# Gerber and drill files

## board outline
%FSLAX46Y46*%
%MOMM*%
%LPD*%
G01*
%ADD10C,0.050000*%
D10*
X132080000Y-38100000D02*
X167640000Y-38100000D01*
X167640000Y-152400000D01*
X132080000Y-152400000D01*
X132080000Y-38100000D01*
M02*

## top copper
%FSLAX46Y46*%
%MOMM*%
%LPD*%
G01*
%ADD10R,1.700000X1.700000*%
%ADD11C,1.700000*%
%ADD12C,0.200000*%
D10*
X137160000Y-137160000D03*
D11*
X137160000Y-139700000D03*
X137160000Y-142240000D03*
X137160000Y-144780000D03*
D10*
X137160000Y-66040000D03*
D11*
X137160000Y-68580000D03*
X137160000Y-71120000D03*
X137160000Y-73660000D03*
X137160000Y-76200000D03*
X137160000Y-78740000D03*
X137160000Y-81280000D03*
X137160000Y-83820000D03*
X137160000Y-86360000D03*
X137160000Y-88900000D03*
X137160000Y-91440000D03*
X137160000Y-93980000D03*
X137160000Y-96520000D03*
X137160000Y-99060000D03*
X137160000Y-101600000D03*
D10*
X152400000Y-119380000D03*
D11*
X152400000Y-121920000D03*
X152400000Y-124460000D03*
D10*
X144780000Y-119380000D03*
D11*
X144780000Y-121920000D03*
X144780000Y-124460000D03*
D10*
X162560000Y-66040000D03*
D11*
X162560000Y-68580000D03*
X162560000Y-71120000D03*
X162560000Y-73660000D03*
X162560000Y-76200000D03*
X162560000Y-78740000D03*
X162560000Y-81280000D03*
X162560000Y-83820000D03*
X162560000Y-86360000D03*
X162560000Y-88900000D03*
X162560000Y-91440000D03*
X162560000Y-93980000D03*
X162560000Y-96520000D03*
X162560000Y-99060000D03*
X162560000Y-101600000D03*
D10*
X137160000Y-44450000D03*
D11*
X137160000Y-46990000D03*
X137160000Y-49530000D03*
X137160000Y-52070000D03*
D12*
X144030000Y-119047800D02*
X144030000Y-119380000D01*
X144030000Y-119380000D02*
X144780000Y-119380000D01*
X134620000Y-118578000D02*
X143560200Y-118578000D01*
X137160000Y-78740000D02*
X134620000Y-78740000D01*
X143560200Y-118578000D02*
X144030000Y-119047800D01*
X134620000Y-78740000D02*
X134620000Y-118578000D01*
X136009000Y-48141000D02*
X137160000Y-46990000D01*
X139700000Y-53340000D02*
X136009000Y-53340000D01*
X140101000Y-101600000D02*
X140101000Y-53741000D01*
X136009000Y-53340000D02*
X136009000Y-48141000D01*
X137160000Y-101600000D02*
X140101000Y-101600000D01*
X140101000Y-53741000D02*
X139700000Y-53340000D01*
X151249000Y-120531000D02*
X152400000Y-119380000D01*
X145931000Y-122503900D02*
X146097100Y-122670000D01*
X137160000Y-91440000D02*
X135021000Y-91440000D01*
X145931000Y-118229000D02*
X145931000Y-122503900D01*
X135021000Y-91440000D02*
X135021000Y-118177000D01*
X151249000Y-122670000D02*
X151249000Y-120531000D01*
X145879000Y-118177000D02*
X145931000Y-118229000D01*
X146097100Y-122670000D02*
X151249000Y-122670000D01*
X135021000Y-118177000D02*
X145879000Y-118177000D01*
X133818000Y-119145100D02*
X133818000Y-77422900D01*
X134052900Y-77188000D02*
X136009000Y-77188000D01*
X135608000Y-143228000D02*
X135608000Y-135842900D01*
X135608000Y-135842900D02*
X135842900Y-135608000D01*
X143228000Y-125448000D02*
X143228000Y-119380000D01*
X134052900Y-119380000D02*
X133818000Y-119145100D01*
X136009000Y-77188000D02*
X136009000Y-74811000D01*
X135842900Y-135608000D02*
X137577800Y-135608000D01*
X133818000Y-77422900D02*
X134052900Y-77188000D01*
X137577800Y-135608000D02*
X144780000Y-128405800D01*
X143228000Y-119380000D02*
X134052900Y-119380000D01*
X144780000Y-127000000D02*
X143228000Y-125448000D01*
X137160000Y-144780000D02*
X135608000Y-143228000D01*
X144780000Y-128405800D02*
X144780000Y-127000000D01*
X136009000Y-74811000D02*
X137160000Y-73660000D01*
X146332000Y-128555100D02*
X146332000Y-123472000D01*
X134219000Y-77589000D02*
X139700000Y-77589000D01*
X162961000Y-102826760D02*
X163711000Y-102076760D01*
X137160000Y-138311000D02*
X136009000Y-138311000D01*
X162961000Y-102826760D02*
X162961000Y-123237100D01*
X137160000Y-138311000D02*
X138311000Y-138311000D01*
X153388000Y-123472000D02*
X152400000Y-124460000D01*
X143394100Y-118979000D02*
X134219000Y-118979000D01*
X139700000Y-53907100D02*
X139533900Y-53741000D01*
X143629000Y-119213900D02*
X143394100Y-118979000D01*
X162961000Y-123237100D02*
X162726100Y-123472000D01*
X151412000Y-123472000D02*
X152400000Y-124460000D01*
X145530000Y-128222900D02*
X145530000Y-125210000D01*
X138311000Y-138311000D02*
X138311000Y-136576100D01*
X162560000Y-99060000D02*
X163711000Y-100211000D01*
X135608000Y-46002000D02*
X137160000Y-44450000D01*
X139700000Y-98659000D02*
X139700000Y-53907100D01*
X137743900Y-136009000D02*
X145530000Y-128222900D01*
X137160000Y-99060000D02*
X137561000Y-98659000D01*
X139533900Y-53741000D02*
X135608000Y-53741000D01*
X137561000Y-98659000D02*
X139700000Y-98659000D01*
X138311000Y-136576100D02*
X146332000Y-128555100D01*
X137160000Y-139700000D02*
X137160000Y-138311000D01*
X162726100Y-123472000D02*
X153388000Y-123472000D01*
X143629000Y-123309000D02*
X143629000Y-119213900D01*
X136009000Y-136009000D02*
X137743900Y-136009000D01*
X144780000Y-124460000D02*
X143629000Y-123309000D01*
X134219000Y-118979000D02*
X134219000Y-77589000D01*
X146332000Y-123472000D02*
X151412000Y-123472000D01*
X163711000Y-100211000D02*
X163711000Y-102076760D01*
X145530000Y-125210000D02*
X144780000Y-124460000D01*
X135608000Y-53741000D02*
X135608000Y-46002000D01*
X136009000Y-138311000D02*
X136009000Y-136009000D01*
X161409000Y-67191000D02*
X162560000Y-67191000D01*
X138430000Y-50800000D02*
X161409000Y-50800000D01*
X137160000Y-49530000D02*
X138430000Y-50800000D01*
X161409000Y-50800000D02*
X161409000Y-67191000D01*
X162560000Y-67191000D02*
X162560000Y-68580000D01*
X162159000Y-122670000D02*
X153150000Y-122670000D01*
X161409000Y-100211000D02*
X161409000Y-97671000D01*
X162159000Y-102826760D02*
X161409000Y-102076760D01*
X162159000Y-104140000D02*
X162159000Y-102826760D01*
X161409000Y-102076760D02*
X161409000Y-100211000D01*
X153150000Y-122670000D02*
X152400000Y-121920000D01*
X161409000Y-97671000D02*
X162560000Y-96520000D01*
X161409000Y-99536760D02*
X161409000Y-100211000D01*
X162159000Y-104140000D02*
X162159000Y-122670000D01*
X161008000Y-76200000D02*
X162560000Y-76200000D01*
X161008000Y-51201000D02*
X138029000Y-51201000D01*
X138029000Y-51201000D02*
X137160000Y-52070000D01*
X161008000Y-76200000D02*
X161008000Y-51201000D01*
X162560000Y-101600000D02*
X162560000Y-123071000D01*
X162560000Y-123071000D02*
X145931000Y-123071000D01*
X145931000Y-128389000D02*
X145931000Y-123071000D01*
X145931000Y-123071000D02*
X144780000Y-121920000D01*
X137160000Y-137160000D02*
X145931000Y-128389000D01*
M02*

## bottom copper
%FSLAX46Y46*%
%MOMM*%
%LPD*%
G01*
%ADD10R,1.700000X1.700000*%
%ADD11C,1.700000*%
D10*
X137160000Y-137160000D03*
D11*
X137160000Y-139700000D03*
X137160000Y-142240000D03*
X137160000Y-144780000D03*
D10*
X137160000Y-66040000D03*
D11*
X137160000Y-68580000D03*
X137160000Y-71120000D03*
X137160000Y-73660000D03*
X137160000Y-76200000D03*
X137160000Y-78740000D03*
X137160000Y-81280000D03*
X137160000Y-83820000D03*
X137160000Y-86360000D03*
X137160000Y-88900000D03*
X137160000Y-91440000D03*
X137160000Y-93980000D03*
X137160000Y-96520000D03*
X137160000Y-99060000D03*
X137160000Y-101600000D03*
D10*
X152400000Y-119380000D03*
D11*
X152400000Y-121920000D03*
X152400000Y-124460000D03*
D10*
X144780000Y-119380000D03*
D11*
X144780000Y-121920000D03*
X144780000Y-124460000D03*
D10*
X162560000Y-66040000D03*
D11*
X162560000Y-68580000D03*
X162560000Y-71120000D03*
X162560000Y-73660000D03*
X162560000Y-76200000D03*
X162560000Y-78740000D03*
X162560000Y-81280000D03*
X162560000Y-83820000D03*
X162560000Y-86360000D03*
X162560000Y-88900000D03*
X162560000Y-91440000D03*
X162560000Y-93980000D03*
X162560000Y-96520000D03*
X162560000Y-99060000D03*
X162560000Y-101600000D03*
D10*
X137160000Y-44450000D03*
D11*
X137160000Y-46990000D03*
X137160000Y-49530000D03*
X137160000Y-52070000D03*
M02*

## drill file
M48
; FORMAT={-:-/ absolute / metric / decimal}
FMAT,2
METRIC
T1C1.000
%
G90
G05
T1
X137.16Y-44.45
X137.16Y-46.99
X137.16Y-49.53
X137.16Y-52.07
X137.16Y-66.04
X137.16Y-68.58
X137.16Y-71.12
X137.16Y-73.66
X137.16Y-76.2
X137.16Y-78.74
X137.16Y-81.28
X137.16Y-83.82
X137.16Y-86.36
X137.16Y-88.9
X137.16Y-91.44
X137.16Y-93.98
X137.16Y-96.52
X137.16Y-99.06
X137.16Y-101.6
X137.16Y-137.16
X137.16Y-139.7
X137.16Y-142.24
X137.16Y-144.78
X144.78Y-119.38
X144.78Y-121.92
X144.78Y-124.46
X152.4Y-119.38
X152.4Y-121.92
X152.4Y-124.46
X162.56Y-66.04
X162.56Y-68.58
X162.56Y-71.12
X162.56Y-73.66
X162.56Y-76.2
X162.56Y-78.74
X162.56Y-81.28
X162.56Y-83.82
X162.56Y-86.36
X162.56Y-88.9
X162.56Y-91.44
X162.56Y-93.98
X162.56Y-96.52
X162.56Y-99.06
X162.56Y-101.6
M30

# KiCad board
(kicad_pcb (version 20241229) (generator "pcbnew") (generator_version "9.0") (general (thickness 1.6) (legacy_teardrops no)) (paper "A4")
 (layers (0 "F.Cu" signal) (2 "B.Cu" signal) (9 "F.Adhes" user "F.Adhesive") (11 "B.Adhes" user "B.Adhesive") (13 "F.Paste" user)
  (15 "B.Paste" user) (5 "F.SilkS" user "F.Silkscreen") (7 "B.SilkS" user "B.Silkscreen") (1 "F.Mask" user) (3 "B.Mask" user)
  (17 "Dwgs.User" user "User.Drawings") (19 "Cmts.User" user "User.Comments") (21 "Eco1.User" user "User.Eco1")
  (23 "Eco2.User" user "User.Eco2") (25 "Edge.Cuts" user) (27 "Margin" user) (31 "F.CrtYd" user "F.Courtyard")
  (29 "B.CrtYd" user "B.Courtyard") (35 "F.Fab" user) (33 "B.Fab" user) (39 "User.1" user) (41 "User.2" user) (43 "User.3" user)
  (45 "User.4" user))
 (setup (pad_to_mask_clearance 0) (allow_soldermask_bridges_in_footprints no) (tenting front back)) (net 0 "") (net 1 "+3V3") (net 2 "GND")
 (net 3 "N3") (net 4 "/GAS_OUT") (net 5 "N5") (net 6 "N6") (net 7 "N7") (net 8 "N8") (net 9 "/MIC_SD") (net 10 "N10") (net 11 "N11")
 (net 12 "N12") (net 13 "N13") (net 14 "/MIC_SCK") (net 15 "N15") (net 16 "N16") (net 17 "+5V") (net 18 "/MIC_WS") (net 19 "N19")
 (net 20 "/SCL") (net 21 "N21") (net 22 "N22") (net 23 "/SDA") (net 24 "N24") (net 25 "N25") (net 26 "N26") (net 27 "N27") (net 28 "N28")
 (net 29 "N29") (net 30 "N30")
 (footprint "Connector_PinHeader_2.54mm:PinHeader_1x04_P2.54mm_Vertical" (layer "F.Cu") (at 137.16 137.16)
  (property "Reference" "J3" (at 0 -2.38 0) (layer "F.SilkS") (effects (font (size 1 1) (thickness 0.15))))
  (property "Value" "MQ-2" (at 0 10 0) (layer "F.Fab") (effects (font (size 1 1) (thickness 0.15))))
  (pad "1" thru_hole rect (at 0 0) (size 1.7 1.7) (drill 1) (layers "*.Cu" "*.Mask") (remove_unused_layers no) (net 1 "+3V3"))
  (pad "2" thru_hole circle (at 0 2.54) (size 1.7 1.7) (drill 1) (layers "*.Cu" "*.Mask") (remove_unused_layers no) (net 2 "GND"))
  (pad "3" thru_hole circle (at 0 5.08) (size 1.7 1.7) (drill 1) (layers "*.Cu" "*.Mask") (remove_unused_layers no) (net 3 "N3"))
  (pad "4" thru_hole circle (at 0 7.62) (size 1.7 1.7) (drill 1) (layers "*.Cu" "*.Mask") (remove_unused_layers no) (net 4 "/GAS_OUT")))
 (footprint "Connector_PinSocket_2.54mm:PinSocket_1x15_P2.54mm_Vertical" (layer "F.Cu") (at 137.16 66.04)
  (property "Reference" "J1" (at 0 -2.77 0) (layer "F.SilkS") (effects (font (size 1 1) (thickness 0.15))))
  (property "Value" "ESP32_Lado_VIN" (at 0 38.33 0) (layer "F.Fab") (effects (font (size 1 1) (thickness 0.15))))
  (pad "1" thru_hole rect (at 0 0) (size 1.7 1.7) (drill 1) (layers "*.Cu" "*.Mask") (remove_unused_layers no) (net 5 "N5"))
  (pad "2" thru_hole circle (at 0 2.54) (size 1.7 1.7) (drill 1) (layers "*.Cu" "*.Mask") (remove_unused_layers no) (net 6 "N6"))
  (pad "3" thru_hole circle (at 0 5.08) (size 1.7 1.7) (drill 1) (layers "*.Cu" "*.Mask") (remove_unused_layers no) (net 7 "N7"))
  (pad "4" thru_hole circle (at 0 7.62) (size 1.7 1.7) (drill 1) (layers "*.Cu" "*.Mask") (remove_unused_layers no) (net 4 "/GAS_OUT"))
  (pad "5" thru_hole circle (at 0 10.16) (size 1.7 1.7) (drill 1) (layers "*.Cu" "*.Mask") (remove_unused_layers no) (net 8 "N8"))
  (pad "6" thru_hole circle (at 0 12.7) (size 1.7 1.7) (drill 1) (layers "*.Cu" "*.Mask") (remove_unused_layers no) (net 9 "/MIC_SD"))
  (pad "7" thru_hole circle (at 0 15.24) (size 1.7 1.7) (drill 1) (layers "*.Cu" "*.Mask") (remove_unused_layers no) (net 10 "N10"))
  (pad "8" thru_hole circle (at 0 17.78) (size 1.7 1.7) (drill 1) (layers "*.Cu" "*.Mask") (remove_unused_layers no) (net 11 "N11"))
  (pad "9" thru_hole circle (at 0 20.32) (size 1.7 1.7) (drill 1) (layers "*.Cu" "*.Mask") (remove_unused_layers no) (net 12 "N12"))
  (pad "10" thru_hole circle (at 0 22.86) (size 1.7 1.7) (drill 1) (layers "*.Cu" "*.Mask") (remove_unused_layers no) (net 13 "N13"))
  (pad "11" thru_hole circle (at 0 25.4) (size 1.7 1.7) (drill 1) (layers "*.Cu" "*.Mask") (remove_unused_layers no) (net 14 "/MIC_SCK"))
  (pad "12" thru_hole circle (at 0 27.94) (size 1.7 1.7) (drill 1) (layers "*.Cu" "*.Mask") (remove_unused_layers no) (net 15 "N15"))
  (pad "13" thru_hole circle (at 0 30.48) (size 1.7 1.7) (drill 1) (layers "*.Cu" "*.Mask") (remove_unused_layers no) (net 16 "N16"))
  (pad "14" thru_hole circle (at 0 33.02) (size 1.7 1.7) (drill 1) (layers "*.Cu" "*.Mask") (remove_unused_layers no) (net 2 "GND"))
  (pad "15" thru_hole circle (at 0 35.56) (size 1.7 1.7) (drill 1) (layers "*.Cu" "*.Mask") (remove_unused_layers no) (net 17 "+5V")))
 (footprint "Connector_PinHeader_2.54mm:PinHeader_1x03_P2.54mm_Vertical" (layer "F.Cu") (at 152.4 119.38)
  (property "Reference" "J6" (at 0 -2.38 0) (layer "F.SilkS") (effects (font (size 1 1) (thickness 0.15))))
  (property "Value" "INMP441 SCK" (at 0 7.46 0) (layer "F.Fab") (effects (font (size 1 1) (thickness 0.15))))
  (pad "1" thru_hole rect (at 0 0) (size 1.7 1.7) (drill 1) (layers "*.Cu" "*.Mask") (remove_unused_layers no) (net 14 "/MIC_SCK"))
  (pad "2" thru_hole circle (at 0 2.54) (size 1.7 1.7) (drill 1) (layers "*.Cu" "*.Mask") (remove_unused_layers no) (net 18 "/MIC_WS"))
  (pad "3" thru_hole circle (at 0 5.08) (size 1.7 1.7) (drill 1) (layers "*.Cu" "*.Mask") (remove_unused_layers no) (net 2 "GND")))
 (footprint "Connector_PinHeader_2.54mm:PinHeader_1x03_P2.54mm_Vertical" (layer "F.Cu") (at 144.78 119.38)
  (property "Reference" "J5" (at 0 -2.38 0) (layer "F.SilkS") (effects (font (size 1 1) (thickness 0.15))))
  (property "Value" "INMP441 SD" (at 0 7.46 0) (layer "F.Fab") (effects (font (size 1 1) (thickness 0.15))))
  (pad "1" thru_hole rect (at 0 0) (size 1.7 1.7) (drill 1) (layers "*.Cu" "*.Mask") (remove_unused_layers no) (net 9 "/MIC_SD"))
  (pad "2" thru_hole circle (at 0 2.54) (size 1.7 1.7) (drill 1) (layers "*.Cu" "*.Mask") (remove_unused_layers no) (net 1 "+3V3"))
  (pad "3" thru_hole circle (at 0 5.08) (size 1.7 1.7) (drill 1) (layers "*.Cu" "*.Mask") (remove_unused_layers no) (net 2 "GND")))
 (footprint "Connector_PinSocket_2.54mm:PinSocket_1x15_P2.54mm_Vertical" (layer "F.Cu") (at 162.56 66.04)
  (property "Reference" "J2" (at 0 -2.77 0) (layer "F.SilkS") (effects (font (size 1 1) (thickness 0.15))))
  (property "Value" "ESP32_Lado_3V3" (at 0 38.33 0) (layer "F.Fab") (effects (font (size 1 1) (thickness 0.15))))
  (pad "1" thru_hole rect (at 0 0) (size 1.7 1.7) (drill 1) (layers "*.Cu" "*.Mask") (remove_unused_layers no) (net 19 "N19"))
  (pad "2" thru_hole circle (at 0 2.54) (size 1.7 1.7) (drill 1) (layers "*.Cu" "*.Mask") (remove_unused_layers no) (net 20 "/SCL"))
  (pad "3" thru_hole circle (at 0 5.08) (size 1.7 1.7) (drill 1) (layers "*.Cu" "*.Mask") (remove_unused_layers no) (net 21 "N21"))
  (pad "4" thru_hole circle (at 0 7.62) (size 1.7 1.7) (drill 1) (layers "*.Cu" "*.Mask") (remove_unused_layers no) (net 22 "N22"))
  (pad "5" thru_hole circle (at 0 10.16) (size 1.7 1.7) (drill 1) (layers "*.Cu" "*.Mask") (remove_unused_layers no) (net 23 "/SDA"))
  (pad "6" thru_hole circle (at 0 12.7) (size 1.7 1.7) (drill 1) (layers "*.Cu" "*.Mask") (remove_unused_layers no) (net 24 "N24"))
  (pad "7" thru_hole circle (at 0 15.24) (size 1.7 1.7) (drill 1) (layers "*.Cu" "*.Mask") (remove_unused_layers no) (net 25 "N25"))
  (pad "8" thru_hole circle (at 0 17.78) (size 1.7 1.7) (drill 1) (layers "*.Cu" "*.Mask") (remove_unused_layers no) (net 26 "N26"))
  (pad "9" thru_hole circle (at 0 20.32) (size 1.7 1.7) (drill 1) (layers "*.Cu" "*.Mask") (remove_unused_layers no) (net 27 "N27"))
  (pad "10" thru_hole circle (at 0 22.86) (size 1.7 1.7) (drill 1) (layers "*.Cu" "*.Mask") (remove_unused_layers no) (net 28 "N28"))
  (pad "11" thru_hole circle (at 0 25.4) (size 1.7 1.7) (drill 1) (layers "*.Cu" "*.Mask") (remove_unused_layers no) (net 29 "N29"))
  (pad "12" thru_hole circle (at 0 27.94) (size 1.7 1.7) (drill 1) (layers "*.Cu" "*.Mask") (remove_unused_layers no) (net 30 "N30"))
  (pad "13" thru_hole circle (at 0 30.48) (size 1.7 1.7) (drill 1) (layers "*.Cu" "*.Mask") (remove_unused_layers no) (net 18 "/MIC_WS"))
  (pad "14" thru_hole circle (at 0 33.02) (size 1.7 1.7) (drill 1) (layers "*.Cu" "*.Mask") (remove_unused_layers no) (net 2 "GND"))
  (pad "15" thru_hole circle (at 0 35.56) (size 1.7 1.7) (drill 1) (layers "*.Cu" "*.Mask") (remove_unused_layers no) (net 1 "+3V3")))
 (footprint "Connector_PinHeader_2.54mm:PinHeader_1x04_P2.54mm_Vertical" (layer "F.Cu") (at 137.16 44.45)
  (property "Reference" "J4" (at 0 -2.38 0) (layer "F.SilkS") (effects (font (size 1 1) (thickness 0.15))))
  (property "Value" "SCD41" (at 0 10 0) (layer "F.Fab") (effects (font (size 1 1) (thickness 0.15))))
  (pad "1" thru_hole rect (at 0 0) (size 1.7 1.7) (drill 1) (layers "*.Cu" "*.Mask") (remove_unused_layers no) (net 2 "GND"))
  (pad "2" thru_hole circle (at 0 2.54) (size 1.7 1.7) (drill 1) (layers "*.Cu" "*.Mask") (remove_unused_layers no) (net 17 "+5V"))
  (pad "3" thru_hole circle (at 0 5.08) (size 1.7 1.7) (drill 1) (layers "*.Cu" "*.Mask") (remove_unused_layers no) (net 20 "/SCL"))
  (pad "4" thru_hole circle (at 0 7.62) (size 1.7 1.7) (drill 1) (layers "*.Cu" "*.Mask") (remove_unused_layers no) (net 23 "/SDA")))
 (gr_rect (start 132.08 38.1) (end 167.64 152.4) (stroke (width 0.05) (type default)) (fill no) (layer "Edge.Cuts"))
 (segment (start 144.03 119.0478) (end 144.03 119.38) (width 0.2) (layer "F.Cu") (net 9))
 (segment (start 144.03 119.38) (end 144.78 119.38) (width 0.2) (layer "F.Cu") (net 9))
 (segment (start 134.62 118.578) (end 143.5602 118.578) (width 0.2) (layer "F.Cu") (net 9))
 (segment (start 137.16 78.74) (end 134.62 78.74) (width 0.2) (layer "F.Cu") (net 9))
 (segment (start 143.5602 118.578) (end 144.03 119.0478) (width 0.2) (layer "F.Cu") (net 9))
 (segment (start 134.62 78.74) (end 134.62 118.578) (width 0.2) (layer "F.Cu") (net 9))
 (segment (start 136.009 48.141) (end 137.16 46.99) (width 0.2) (layer "F.Cu") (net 17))
 (segment (start 139.7 53.34) (end 136.009 53.34) (width 0.2) (layer "F.Cu") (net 17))
 (segment (start 140.101 101.6) (end 140.101 53.741) (width 0.2) (layer "F.Cu") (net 17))
 (segment (start 136.009 53.34) (end 136.009 48.141) (width 0.2) (layer "F.Cu") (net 17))
 (segment (start 137.16 101.6) (end 140.101 101.6) (width 0.2) (layer "F.Cu") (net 17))
 (segment (start 140.101 53.741) (end 139.7 53.34) (width 0.2) (layer "F.Cu") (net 17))
 (segment (start 151.249 120.531) (end 152.4 119.38) (width 0.2) (layer "F.Cu") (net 14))
 (segment (start 145.931 122.5039) (end 146.0971 122.67) (width 0.2) (layer "F.Cu") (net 14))
 (segment (start 137.16 91.44) (end 135.021 91.44) (width 0.2) (layer "F.Cu") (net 14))
 (segment (start 145.931 118.229) (end 145.931 122.5039) (width 0.2) (layer "F.Cu") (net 14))
 (segment (start 135.021 91.44) (end 135.021 118.177) (width 0.2) (layer "F.Cu") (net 14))
 (segment (start 151.249 122.67) (end 151.249 120.531) (width 0.2) (layer "F.Cu") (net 14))
 (segment (start 145.879 118.177) (end 145.931 118.229) (width 0.2) (layer "F.Cu") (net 14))
 (segment (start 146.0971 122.67) (end 151.249 122.67) (width 0.2) (layer "F.Cu") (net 14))
 (segment (start 135.021 118.177) (end 145.879 118.177) (width 0.2) (layer "F.Cu") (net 14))
 (segment (start 133.818 119.1451) (end 133.818 77.4229) (width 0.2) (layer "F.Cu") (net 4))
 (segment (start 134.0529 77.188) (end 136.009 77.188) (width 0.2) (layer "F.Cu") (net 4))
 (segment (start 135.608 143.228) (end 135.608 135.8429) (width 0.2) (layer "F.Cu") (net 4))
 (segment (start 135.608 135.8429) (end 135.8429 135.608) (width 0.2) (layer "F.Cu") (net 4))
 (segment (start 143.228 125.448) (end 143.228 119.38) (width 0.2) (layer "F.Cu") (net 4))
 (segment (start 134.0529 119.38) (end 133.818 119.1451) (width 0.2) (layer "F.Cu") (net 4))
 (segment (start 136.009 77.188) (end 136.009 74.811) (width 0.2) (layer "F.Cu") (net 4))
 (segment (start 135.8429 135.608) (end 137.5778 135.608) (width 0.2) (layer "F.Cu") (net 4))
 (segment (start 133.818 77.4229) (end 134.0529 77.188) (width 0.2) (layer "F.Cu") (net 4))
 (segment (start 137.5778 135.608) (end 144.78 128.4058) (width 0.2) (layer "F.Cu") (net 4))
 (segment (start 143.228 119.38) (end 134.0529 119.38) (width 0.2) (layer "F.Cu") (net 4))
 (segment (start 144.78 127) (end 143.228 125.448) (width 0.2) (layer "F.Cu") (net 4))
 (segment (start 137.16 144.78) (end 135.608 143.228) (width 0.2) (layer "F.Cu") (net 4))
 (segment (start 144.78 128.4058) (end 144.78 127) (width 0.2) (layer "F.Cu") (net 4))
 (segment (start 136.009 74.811) (end 137.16 73.66) (width 0.2) (layer "F.Cu") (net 4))
 (segment (start 146.332 128.5551) (end 146.332 123.472) (width 0.2) (layer "F.Cu") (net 2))
 (segment (start 134.219 77.589) (end 139.7 77.589) (width 0.2) (layer "F.Cu") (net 2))
 (segment (start 162.961 102.82676) (end 163.711 102.07676) (width 0.2) (layer "F.Cu") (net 2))
 (segment (start 137.16 138.311) (end 136.009 138.311) (width 0.2) (layer "F.Cu") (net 2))
 (segment (start 162.961 102.82676) (end 162.961 123.2371) (width 0.2) (layer "F.Cu") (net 2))
 (segment (start 137.16 138.311) (end 138.311 138.311) (width 0.2) (layer "F.Cu") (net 2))
 (segment (start 153.388 123.472) (end 152.4 124.46) (width 0.2) (layer "F.Cu") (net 2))
 (segment (start 143.3941 118.979) (end 134.219 118.979) (width 0.2) (layer "F.Cu") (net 2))
 (segment (start 139.7 53.9071) (end 139.5339 53.741) (width 0.2) (layer "F.Cu") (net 2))
 (segment (start 143.629 119.2139) (end 143.3941 118.979) (width 0.2) (layer "F.Cu") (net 2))
 (segment (start 162.961 123.2371) (end 162.7261 123.472) (width 0.2) (layer "F.Cu") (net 2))
 (segment (start 151.412 123.472) (end 152.4 124.46) (width 0.2) (layer "F.Cu") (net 2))
 (segment (start 145.53 128.2229) (end 145.53 125.21) (width 0.2) (layer "F.Cu") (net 2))
 (segment (start 138.311 138.311) (end 138.311 136.5761) (width 0.2) (layer "F.Cu") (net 2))
 (segment (start 162.56 99.06) (end 163.711 100.211) (width 0.2) (layer "F.Cu") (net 2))
 (segment (start 135.608 46.002) (end 137.16 44.45) (width 0.2) (layer "F.Cu") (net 2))
 (segment (start 139.7 98.659) (end 139.7 53.9071) (width 0.2) (layer "F.Cu") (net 2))
 (segment (start 137.7439 136.009) (end 145.53 128.2229) (width 0.2) (layer "F.Cu") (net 2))
 (segment (start 137.16 99.06) (end 137.561 98.659) (width 0.2) (layer "F.Cu") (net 2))
 (segment (start 139.5339 53.741) (end 135.608 53.741) (width 0.2) (layer "F.Cu") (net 2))
 (segment (start 137.561 98.659) (end 139.7 98.659) (width 0.2) (layer "F.Cu") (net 2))
 (segment (start 138.311 136.5761) (end 146.332 128.5551) (width 0.2) (layer "F.Cu") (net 2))
 (segment (start 137.16 139.7) (end 137.16 138.311) (width 0.2) (layer "F.Cu") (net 2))
 (segment (start 162.7261 123.472) (end 153.388 123.472) (width 0.2) (layer "F.Cu") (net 2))
 (segment (start 143.629 123.309) (end 143.629 119.2139) (width 0.2) (layer "F.Cu") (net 2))
 (segment (start 136.009 136.009) (end 137.7439 136.009) (width 0.2) (layer "F.Cu") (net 2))
 (segment (start 144.78 124.46) (end 143.629 123.309) (width 0.2) (layer "F.Cu") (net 2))
 (segment (start 134.219 118.979) (end 134.219 77.589) (width 0.2) (layer "F.Cu") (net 2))
 (segment (start 146.332 123.472) (end 151.412 123.472) (width 0.2) (layer "F.Cu") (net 2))
 (segment (start 163.711 100.211) (end 163.711 102.07676) (width 0.2) (layer "F.Cu") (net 2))
 (segment (start 145.53 125.21) (end 144.78 124.46) (width 0.2) (layer "F.Cu") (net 2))
 (segment (start 135.608 53.741) (end 135.608 46.002) (width 0.2) (layer "F.Cu") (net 2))
 (segment (start 136.009 138.311) (end 136.009 136.009) (width 0.2) (layer "F.Cu") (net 2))
 (segment (start 161.409 67.191) (end 162.56 67.191) (width 0.2) (layer "F.Cu") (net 20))
 (segment (start 138.43 50.8) (end 161.409 50.8) (width 0.2) (layer "F.Cu") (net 20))
 (segment (start 137.16 49.53) (end 138.43 50.8) (width 0.2) (layer "F.Cu") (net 20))
 (segment (start 161.409 50.8) (end 161.409 67.191) (width 0.2) (layer "F.Cu") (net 20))
 (segment (start 162.56 67.191) (end 162.56 68.58) (width 0.2) (layer "F.Cu") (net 20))
 (segment (start 162.159 122.67) (end 153.15 122.67) (width 0.2) (layer "F.Cu") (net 18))
 (segment (start 161.409 100.211) (end 161.409 97.671) (width 0.2) (layer "F.Cu") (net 18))
 (segment (start 162.159 102.82676) (end 161.409 102.07676) (width 0.2) (layer "F.Cu") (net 18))
 (segment (start 162.159 104.14) (end 162.159 102.82676) (width 0.2) (layer "F.Cu") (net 18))
 (segment (start 161.409 102.07676) (end 161.409 100.211) (width 0.2) (layer "F.Cu") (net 18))
 (segment (start 153.15 122.67) (end 152.4 121.92) (width 0.2) (layer "F.Cu") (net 18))
 (segment (start 161.409 97.671) (end 162.56 96.52) (width 0.2) (layer "F.Cu") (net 18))
 (segment (start 161.409 99.53676) (end 161.409 100.211) (width 0.2) (layer "F.Cu") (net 18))
 (segment (start 162.159 104.14) (end 162.159 122.67) (width 0.2) (layer "F.Cu") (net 18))
 (segment (start 161.008 76.2) (end 162.56 76.2) (width 0.2) (layer "F.Cu") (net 23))
 (segment (start 161.008 51.201) (end 138.029 51.201) (width 0.2) (layer "F.Cu") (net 23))
 (segment (start 138.029 51.201) (end 137.16 52.07) (width 0.2) (layer "F.Cu") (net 23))
 (segment (start 161.008 76.2) (end 161.008 51.201) (width 0.2) (layer "F.Cu") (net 23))
 (segment (start 162.56 101.6) (end 162.56 123.071) (width 0.2) (layer "F.Cu") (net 1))
 (segment (start 162.56 123.071) (end 145.931 123.071) (width 0.2) (layer "F.Cu") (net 1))
 (segment (start 145.931 128.389) (end 145.931 123.071) (width 0.2) (layer "F.Cu") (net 1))
 (segment (start 145.931 123.071) (end 144.78 121.92) (width 0.2) (layer "F.Cu") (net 1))
 (segment (start 137.16 137.16) (end 145.931 128.389) (width 0.2) (layer "F.Cu") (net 1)))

